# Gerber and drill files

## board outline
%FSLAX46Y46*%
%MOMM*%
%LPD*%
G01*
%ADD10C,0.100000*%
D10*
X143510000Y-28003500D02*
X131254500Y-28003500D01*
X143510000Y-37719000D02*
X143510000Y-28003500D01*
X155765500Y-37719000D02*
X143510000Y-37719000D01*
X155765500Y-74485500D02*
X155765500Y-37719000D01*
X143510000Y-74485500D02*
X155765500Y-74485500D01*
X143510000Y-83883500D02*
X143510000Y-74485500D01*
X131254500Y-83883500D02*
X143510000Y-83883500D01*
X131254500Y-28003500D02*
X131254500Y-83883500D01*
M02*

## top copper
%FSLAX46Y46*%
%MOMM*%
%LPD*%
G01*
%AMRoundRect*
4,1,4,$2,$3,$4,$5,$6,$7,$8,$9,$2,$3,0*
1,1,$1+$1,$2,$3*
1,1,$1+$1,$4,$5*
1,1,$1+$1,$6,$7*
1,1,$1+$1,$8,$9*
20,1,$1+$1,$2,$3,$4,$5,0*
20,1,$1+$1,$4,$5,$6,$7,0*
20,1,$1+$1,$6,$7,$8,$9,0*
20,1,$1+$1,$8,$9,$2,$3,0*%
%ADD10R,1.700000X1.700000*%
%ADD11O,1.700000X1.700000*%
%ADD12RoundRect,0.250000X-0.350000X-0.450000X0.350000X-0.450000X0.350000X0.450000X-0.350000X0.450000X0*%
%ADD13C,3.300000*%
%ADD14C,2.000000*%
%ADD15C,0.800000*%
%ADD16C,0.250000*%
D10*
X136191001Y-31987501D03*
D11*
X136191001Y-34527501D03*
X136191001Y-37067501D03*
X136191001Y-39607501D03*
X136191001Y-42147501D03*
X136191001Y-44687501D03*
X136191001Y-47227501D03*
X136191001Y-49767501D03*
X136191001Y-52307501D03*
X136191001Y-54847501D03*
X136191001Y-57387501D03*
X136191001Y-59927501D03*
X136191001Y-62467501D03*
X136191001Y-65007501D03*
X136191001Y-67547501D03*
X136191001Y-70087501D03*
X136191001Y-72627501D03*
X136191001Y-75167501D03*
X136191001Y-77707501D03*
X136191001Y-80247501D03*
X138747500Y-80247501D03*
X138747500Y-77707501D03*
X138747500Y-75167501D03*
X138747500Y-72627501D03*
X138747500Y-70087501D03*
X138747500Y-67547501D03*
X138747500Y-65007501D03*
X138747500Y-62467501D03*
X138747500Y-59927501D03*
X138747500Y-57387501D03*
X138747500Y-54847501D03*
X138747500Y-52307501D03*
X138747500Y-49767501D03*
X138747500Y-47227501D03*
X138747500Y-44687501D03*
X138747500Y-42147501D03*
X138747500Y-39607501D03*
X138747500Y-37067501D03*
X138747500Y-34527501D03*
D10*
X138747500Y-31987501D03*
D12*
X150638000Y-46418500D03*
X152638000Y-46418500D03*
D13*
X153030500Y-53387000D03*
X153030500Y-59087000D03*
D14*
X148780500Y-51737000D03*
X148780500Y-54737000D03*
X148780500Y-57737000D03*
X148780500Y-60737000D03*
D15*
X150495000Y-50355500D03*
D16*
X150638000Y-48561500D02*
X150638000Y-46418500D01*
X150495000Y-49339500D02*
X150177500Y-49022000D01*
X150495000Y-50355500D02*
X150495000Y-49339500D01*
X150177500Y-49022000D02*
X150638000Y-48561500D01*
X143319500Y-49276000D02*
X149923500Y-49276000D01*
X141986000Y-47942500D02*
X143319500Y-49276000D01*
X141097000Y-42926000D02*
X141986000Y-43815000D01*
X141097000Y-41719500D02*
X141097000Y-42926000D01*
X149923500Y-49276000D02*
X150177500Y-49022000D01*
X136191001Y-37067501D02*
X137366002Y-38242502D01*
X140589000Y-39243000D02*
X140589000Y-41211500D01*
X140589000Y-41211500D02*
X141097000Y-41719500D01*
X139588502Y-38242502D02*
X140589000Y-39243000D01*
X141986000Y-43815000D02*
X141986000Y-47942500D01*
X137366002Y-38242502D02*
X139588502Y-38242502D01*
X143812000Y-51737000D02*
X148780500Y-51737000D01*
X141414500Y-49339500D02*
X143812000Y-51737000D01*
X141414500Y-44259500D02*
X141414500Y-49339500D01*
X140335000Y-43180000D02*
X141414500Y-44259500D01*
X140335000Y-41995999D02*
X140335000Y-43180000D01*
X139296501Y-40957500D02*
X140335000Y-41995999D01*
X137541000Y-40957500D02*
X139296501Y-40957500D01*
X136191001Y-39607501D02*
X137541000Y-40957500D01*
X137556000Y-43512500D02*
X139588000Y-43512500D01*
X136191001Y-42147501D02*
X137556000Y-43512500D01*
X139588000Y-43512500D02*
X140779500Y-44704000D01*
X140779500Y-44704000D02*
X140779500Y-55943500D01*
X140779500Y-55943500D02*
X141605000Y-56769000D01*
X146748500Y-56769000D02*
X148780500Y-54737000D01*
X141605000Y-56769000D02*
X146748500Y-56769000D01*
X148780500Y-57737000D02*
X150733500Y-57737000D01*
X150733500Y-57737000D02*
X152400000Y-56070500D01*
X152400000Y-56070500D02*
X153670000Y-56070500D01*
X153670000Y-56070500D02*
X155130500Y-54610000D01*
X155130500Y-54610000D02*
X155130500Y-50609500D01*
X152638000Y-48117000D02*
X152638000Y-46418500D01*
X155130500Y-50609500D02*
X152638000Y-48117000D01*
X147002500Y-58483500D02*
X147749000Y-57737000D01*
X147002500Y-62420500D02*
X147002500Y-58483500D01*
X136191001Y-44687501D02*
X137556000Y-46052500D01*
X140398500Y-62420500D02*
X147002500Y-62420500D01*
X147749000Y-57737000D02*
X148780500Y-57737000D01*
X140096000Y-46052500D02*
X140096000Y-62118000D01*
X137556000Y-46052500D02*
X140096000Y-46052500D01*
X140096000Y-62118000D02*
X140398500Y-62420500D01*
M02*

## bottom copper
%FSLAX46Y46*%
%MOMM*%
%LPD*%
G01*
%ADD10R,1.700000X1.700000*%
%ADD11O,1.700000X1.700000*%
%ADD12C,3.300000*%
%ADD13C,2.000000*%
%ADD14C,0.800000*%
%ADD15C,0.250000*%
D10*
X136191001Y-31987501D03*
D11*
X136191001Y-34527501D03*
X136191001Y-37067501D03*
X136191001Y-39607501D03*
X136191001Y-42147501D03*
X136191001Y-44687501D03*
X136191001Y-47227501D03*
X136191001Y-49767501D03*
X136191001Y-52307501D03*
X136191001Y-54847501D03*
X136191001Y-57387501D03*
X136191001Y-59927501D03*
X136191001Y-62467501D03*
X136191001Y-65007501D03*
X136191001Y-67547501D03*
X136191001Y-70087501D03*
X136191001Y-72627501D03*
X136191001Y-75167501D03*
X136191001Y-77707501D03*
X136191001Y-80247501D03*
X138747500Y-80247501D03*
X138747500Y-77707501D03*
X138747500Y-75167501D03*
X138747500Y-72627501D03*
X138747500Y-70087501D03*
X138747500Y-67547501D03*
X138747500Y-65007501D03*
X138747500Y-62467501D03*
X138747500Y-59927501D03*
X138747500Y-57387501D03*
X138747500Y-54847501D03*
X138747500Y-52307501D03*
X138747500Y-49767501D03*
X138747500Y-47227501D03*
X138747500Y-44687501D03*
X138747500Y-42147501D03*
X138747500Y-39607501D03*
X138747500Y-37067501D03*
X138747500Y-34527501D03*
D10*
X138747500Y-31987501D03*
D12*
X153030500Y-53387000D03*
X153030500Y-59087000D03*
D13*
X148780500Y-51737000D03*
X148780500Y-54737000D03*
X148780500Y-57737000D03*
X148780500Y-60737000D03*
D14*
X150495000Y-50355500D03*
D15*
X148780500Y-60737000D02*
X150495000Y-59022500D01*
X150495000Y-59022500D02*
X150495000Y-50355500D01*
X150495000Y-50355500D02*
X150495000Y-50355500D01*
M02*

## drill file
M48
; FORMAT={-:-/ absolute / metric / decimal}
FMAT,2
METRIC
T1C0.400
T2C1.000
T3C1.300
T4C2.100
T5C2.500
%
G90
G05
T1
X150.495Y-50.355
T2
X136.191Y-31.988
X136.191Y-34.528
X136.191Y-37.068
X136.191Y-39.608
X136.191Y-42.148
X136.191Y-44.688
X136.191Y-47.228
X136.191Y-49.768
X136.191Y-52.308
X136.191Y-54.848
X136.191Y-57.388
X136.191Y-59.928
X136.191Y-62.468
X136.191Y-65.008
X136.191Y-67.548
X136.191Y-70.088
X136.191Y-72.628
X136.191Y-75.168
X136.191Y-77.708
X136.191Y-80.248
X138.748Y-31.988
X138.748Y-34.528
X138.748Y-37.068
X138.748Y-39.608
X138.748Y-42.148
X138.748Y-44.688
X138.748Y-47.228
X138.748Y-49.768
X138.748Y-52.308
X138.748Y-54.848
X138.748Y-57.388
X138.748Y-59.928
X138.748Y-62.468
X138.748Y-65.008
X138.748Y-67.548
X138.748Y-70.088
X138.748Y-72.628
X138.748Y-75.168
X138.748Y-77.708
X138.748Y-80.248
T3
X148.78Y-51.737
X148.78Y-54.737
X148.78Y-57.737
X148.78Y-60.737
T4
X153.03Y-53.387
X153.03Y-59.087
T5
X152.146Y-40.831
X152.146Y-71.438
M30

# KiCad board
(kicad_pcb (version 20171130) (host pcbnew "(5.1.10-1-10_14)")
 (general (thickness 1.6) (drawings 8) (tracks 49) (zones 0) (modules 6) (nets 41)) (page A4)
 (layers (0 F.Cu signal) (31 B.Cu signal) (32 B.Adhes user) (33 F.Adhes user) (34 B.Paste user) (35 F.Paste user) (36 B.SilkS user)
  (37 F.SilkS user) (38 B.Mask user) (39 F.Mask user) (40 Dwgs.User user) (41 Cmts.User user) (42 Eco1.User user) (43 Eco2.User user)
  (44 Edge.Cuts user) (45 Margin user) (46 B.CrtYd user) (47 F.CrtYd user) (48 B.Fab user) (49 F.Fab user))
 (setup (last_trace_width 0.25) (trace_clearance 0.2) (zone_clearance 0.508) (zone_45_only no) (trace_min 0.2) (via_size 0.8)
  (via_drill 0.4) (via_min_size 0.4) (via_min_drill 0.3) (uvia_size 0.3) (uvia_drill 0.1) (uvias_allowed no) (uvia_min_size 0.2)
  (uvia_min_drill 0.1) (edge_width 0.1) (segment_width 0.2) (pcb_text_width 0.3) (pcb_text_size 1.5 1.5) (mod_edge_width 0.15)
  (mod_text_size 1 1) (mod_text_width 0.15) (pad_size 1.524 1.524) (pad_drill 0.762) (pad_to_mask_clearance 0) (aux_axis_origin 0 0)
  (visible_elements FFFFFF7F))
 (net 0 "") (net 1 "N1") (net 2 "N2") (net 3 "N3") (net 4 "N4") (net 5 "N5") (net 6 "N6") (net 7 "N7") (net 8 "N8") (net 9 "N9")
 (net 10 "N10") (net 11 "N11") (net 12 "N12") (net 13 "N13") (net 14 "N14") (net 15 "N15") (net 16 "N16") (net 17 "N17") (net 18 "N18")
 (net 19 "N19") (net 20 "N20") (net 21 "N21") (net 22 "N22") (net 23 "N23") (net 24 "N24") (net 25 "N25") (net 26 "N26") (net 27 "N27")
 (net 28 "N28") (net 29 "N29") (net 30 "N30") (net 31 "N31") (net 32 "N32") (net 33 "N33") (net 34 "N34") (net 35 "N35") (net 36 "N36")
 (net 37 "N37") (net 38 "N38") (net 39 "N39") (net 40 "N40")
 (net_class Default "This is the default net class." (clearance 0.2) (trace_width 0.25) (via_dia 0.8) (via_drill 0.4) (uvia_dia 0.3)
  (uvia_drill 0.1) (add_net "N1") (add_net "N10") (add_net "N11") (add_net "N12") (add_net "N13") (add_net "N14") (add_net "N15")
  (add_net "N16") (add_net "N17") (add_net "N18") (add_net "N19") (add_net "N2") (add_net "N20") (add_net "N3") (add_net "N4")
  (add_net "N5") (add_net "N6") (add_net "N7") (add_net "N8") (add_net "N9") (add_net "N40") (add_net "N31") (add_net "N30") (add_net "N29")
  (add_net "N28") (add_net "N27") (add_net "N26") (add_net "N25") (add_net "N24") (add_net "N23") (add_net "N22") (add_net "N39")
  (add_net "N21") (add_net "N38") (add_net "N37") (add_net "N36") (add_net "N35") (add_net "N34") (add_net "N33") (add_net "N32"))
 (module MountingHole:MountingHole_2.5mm (layer F.Cu) (at 152.146 71.4375)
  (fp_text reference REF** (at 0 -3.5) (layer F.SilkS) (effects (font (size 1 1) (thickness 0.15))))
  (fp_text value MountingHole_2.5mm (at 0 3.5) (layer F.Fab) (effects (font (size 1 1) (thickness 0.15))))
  (pad 1 np_thru_hole circle (at 0 0) (size 2.5 2.5) (drill 2.5) (layers *.Cu *.Mask)))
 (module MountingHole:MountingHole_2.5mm (layer F.Cu) (at 152.146 40.8305)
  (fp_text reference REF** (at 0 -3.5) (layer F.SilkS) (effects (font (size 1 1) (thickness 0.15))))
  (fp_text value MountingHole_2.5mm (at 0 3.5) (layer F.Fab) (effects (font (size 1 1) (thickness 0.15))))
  (pad 1 np_thru_hole circle (at 0 0) (size 2.5 2.5) (drill 2.5) (layers *.Cu *.Mask)))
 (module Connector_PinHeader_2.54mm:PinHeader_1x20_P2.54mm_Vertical (layer F.Cu) (at 136.191001 31.987501)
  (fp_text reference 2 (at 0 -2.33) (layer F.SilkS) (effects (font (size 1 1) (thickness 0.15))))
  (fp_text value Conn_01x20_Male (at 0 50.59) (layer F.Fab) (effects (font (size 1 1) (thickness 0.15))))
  (pad 1 thru_hole rect (at 0 0) (size 1.7 1.7) (drill 1) (layers *.Cu *.Mask) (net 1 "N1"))
  (pad 2 thru_hole oval (at 0 2.54) (size 1.7 1.7) (drill 1) (layers *.Cu *.Mask) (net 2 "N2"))
  (pad 3 thru_hole oval (at 0 5.08) (size 1.7 1.7) (drill 1) (layers *.Cu *.Mask) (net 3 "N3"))
  (pad 4 thru_hole oval (at 0 7.62) (size 1.7 1.7) (drill 1) (layers *.Cu *.Mask) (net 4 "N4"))
  (pad 5 thru_hole oval (at 0 10.16) (size 1.7 1.7) (drill 1) (layers *.Cu *.Mask) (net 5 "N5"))
  (pad 6 thru_hole oval (at 0 12.7) (size 1.7 1.7) (drill 1) (layers *.Cu *.Mask) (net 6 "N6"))
  (pad 7 thru_hole oval (at 0 15.24) (size 1.7 1.7) (drill 1) (layers *.Cu *.Mask) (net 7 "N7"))
  (pad 8 thru_hole oval (at 0 17.78) (size 1.7 1.7) (drill 1) (layers *.Cu *.Mask) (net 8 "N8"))
  (pad 9 thru_hole oval (at 0 20.32) (size 1.7 1.7) (drill 1) (layers *.Cu *.Mask) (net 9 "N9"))
  (pad 10 thru_hole oval (at 0 22.86) (size 1.7 1.7) (drill 1) (layers *.Cu *.Mask) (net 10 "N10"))
  (pad 11 thru_hole oval (at 0 25.4) (size 1.7 1.7) (drill 1) (layers *.Cu *.Mask) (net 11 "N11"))
  (pad 12 thru_hole oval (at 0 27.94) (size 1.7 1.7) (drill 1) (layers *.Cu *.Mask) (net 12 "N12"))
  (pad 13 thru_hole oval (at 0 30.48) (size 1.7 1.7) (drill 1) (layers *.Cu *.Mask) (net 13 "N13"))
  (pad 14 thru_hole oval (at 0 33.02) (size 1.7 1.7) (drill 1) (layers *.Cu *.Mask) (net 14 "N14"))
  (pad 15 thru_hole oval (at 0 35.56) (size 1.7 1.7) (drill 1) (layers *.Cu *.Mask) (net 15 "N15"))
  (pad 16 thru_hole oval (at 0 38.1) (size 1.7 1.7) (drill 1) (layers *.Cu *.Mask) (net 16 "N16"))
  (pad 17 thru_hole oval (at 0 40.64) (size 1.7 1.7) (drill 1) (layers *.Cu *.Mask) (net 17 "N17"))
  (pad 18 thru_hole oval (at 0 43.18) (size 1.7 1.7) (drill 1) (layers *.Cu *.Mask) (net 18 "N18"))
  (pad 19 thru_hole oval (at 0 45.72) (size 1.7 1.7) (drill 1) (layers *.Cu *.Mask) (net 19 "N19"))
  (pad 20 thru_hole oval (at 0 48.26) (size 1.7 1.7) (drill 1) (layers *.Cu *.Mask) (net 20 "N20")))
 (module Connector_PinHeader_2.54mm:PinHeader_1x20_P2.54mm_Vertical (layer F.Cu) (at 138.7475 31.987501)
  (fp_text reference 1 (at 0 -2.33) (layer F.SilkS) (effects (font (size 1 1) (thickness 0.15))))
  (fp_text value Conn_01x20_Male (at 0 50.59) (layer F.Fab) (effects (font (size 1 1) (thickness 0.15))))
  (pad 20 thru_hole oval (at 0 48.26) (size 1.7 1.7) (drill 1) (layers *.Cu *.Mask) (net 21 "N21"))
  (pad 19 thru_hole oval (at 0 45.72) (size 1.7 1.7) (drill 1) (layers *.Cu *.Mask) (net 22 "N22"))
  (pad 18 thru_hole oval (at 0 43.18) (size 1.7 1.7) (drill 1) (layers *.Cu *.Mask) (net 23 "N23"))
  (pad 17 thru_hole oval (at 0 40.64) (size 1.7 1.7) (drill 1) (layers *.Cu *.Mask) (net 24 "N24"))
  (pad 16 thru_hole oval (at 0 38.1) (size 1.7 1.7) (drill 1) (layers *.Cu *.Mask) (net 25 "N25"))
  (pad 15 thru_hole oval (at 0 35.56) (size 1.7 1.7) (drill 1) (layers *.Cu *.Mask) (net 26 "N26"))
  (pad 14 thru_hole oval (at 0 33.02) (size 1.7 1.7) (drill 1) (layers *.Cu *.Mask) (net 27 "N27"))
  (pad 13 thru_hole oval (at 0 30.48) (size 1.7 1.7) (drill 1) (layers *.Cu *.Mask) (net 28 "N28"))
  (pad 12 thru_hole oval (at 0 27.94) (size 1.7 1.7) (drill 1) (layers *.Cu *.Mask) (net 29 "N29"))
  (pad 11 thru_hole oval (at 0 25.4) (size 1.7 1.7) (drill 1) (layers *.Cu *.Mask) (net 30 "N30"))
  (pad 10 thru_hole oval (at 0 22.86) (size 1.7 1.7) (drill 1) (layers *.Cu *.Mask) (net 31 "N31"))
  (pad 9 thru_hole oval (at 0 20.32) (size 1.7 1.7) (drill 1) (layers *.Cu *.Mask) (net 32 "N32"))
  (pad 8 thru_hole oval (at 0 17.78) (size 1.7 1.7) (drill 1) (layers *.Cu *.Mask) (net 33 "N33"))
  (pad 7 thru_hole oval (at 0 15.24) (size 1.7 1.7) (drill 1) (layers *.Cu *.Mask) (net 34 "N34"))
  (pad 6 thru_hole oval (at 0 12.7) (size 1.7 1.7) (drill 1) (layers *.Cu *.Mask) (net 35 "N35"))
  (pad 5 thru_hole oval (at 0 10.16) (size 1.7 1.7) (drill 1) (layers *.Cu *.Mask) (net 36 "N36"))
  (pad 4 thru_hole oval (at 0 7.62) (size 1.7 1.7) (drill 1) (layers *.Cu *.Mask) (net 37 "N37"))
  (pad 3 thru_hole oval (at 0 5.08) (size 1.7 1.7) (drill 1) (layers *.Cu *.Mask) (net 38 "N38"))
  (pad 2 thru_hole oval (at 0 2.54) (size 1.7 1.7) (drill 1) (layers *.Cu *.Mask) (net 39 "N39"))
  (pad 1 thru_hole rect (at 0 0) (size 1.7 1.7) (drill 1) (layers *.Cu *.Mask) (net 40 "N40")))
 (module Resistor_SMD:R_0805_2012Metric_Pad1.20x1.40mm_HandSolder (layer F.Cu) (at 151.638 46.4185)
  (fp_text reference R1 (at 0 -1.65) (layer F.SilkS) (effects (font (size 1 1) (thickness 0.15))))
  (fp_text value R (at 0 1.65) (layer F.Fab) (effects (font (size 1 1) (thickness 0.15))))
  (pad 1 smd roundrect (at -1 0) (size 1.2 1.4) (layers F.Cu F.Paste F.Mask) (roundrect_rratio 0.208333) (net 3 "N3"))
  (pad 2 smd roundrect (at 1 0) (size 1.2 1.4) (layers F.Cu F.Paste F.Mask) (roundrect_rratio 0.208333) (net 6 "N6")))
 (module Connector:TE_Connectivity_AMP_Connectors (layer B.Cu) (at 153.0305 53.887 270)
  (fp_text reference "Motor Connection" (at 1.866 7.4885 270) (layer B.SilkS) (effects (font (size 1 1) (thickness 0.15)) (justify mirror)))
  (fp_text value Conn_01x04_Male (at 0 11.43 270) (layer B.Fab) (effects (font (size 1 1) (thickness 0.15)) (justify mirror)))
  (pad 5 thru_hole circle (at -0.5 0 270) (size 3.3 3.3) (drill 2.1) (layers *.Cu *.Mask))
  (pad 6 thru_hole circle (at 5.2 0 270) (size 3.3 3.3) (drill 2.1) (layers *.Cu *.Mask))
  (pad 1 thru_hole circle (at -2.15 4.25 270) (size 2 2) (drill 1.3) (layers *.Cu *.Mask) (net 4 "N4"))
  (pad 2 thru_hole circle (at 0.85 4.25 270) (size 2 2) (drill 1.3) (layers *.Cu *.Mask) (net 5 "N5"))
  (pad 3 thru_hole circle (at 3.85 4.25 270) (size 2 2) (drill 1.3) (layers *.Cu *.Mask) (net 6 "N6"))
  (pad 4 thru_hole circle (at 6.85 4.25 270) (size 2 2) (drill 1.3) (layers *.Cu *.Mask) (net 3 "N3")))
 (gr_line (start 143.51 28.0035) (end 131.2545 28.0035) (layer Edge.Cuts) (width 0.1))
 (gr_line (start 143.51 37.719) (end 143.51 28.0035) (layer Edge.Cuts) (width 0.1))
 (gr_line (start 155.7655 37.719) (end 143.51 37.719) (layer Edge.Cuts) (width 0.1))
 (gr_line (start 155.7655 74.4855) (end 155.7655 37.719) (layer Edge.Cuts) (width 0.1))
 (gr_line (start 143.51 74.4855) (end 155.7655 74.4855) (layer Edge.Cuts) (width 0.1))
 (gr_line (start 143.51 83.8835) (end 143.51 74.4855) (layer Edge.Cuts) (width 0.1))
 (gr_line (start 131.2545 83.8835) (end 143.51 83.8835) (layer Edge.Cuts) (width 0.1))
 (gr_line (start 131.2545 28.0035) (end 131.2545 83.8835) (layer Edge.Cuts) (width 0.1))
 (segment (start 150.638 48.5615) (end 150.638 46.4185) (width 0.25) (layer F.Cu) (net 3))
 (segment (start 148.7805 60.737) (end 150.495 59.0225) (width 0.25) (layer B.Cu) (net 3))
 (segment (start 150.495 59.0225) (end 150.495 50.3555) (width 0.25) (layer B.Cu) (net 3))
 (segment (start 150.495 50.3555) (end 150.495 50.3555) (width 0.25) (layer B.Cu) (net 3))
 (via (at 150.495 50.3555) (size 0.8) (drill 0.4) (layers F.Cu B.Cu) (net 3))
 (segment (start 150.495 49.3395) (end 150.1775 49.022) (width 0.25) (layer F.Cu) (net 3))
 (segment (start 150.495 50.3555) (end 150.495 49.3395) (width 0.25) (layer F.Cu) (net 3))
 (segment (start 150.1775 49.022) (end 150.638 48.5615) (width 0.25) (layer F.Cu) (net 3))
 (segment (start 143.3195 49.276) (end 149.9235 49.276) (width 0.25) (layer F.Cu) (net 3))
 (segment (start 141.986 47.9425) (end 143.3195 49.276) (width 0.25) (layer F.Cu) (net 3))
 (segment (start 141.097 42.926) (end 141.986 43.815) (width 0.25) (layer F.Cu) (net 3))
 (segment (start 141.097 41.7195) (end 141.097 42.926) (width 0.25) (layer F.Cu) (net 3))
 (segment (start 149.9235 49.276) (end 150.1775 49.022) (width 0.25) (layer F.Cu) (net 3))
 (segment (start 136.191001 37.067501) (end 137.366002 38.242502) (width 0.25) (layer F.Cu) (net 3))
 (segment (start 140.589 39.243) (end 140.589 41.2115) (width 0.25) (layer F.Cu) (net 3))
 (segment (start 140.589 41.2115) (end 141.097 41.7195) (width 0.25) (layer F.Cu) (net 3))
 (segment (start 139.588502 38.242502) (end 140.589 39.243) (width 0.25) (layer F.Cu) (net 3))
 (segment (start 141.986 43.815) (end 141.986 47.9425) (width 0.25) (layer F.Cu) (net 3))
 (segment (start 137.366002 38.242502) (end 139.588502 38.242502) (width 0.25) (layer F.Cu) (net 3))
 (segment (start 143.812 51.737) (end 148.7805 51.737) (width 0.25) (layer F.Cu) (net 4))
 (segment (start 141.4145 49.3395) (end 143.812 51.737) (width 0.25) (layer F.Cu) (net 4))
 (segment (start 141.4145 44.2595) (end 141.4145 49.3395) (width 0.25) (layer F.Cu) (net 4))
 (segment (start 140.335 43.18) (end 141.4145 44.2595) (width 0.25) (layer F.Cu) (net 4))
 (segment (start 140.335 41.995999) (end 140.335 43.18) (width 0.25) (layer F.Cu) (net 4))
 (segment (start 139.296501 40.9575) (end 140.335 41.995999) (width 0.25) (layer F.Cu) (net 4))
 (segment (start 137.541 40.9575) (end 139.296501 40.9575) (width 0.25) (layer F.Cu) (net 4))
 (segment (start 136.191001 39.607501) (end 137.541 40.9575) (width 0.25) (layer F.Cu) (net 4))
 (segment (start 137.556 43.5125) (end 139.588 43.5125) (width 0.25) (layer F.Cu) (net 5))
 (segment (start 136.191001 42.147501) (end 137.556 43.5125) (width 0.25) (layer F.Cu) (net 5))
 (segment (start 139.588 43.5125) (end 140.7795 44.704) (width 0.25) (layer F.Cu) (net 5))
 (segment (start 140.7795 44.704) (end 140.7795 55.9435) (width 0.25) (layer F.Cu) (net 5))
 (segment (start 140.7795 55.9435) (end 141.605 56.769) (width 0.25) (layer F.Cu) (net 5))
 (segment (start 146.7485 56.769) (end 148.7805 54.737) (width 0.25) (layer F.Cu) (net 5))
 (segment (start 141.605 56.769) (end 146.7485 56.769) (width 0.25) (layer F.Cu) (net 5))
 (segment (start 148.7805 57.737) (end 150.7335 57.737) (width 0.25) (layer F.Cu) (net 6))
 (segment (start 150.7335 57.737) (end 152.4 56.0705) (width 0.25) (layer F.Cu) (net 6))
 (segment (start 152.4 56.0705) (end 153.67 56.0705) (width 0.25) (layer F.Cu) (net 6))
 (segment (start 153.67 56.0705) (end 155.1305 54.61) (width 0.25) (layer F.Cu) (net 6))
 (segment (start 155.1305 54.61) (end 155.1305 50.6095) (width 0.25) (layer F.Cu) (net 6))
 (segment (start 152.638 48.117) (end 152.638 46.4185) (width 0.25) (layer F.Cu) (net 6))
 (segment (start 155.1305 50.6095) (end 152.638 48.117) (width 0.25) (layer F.Cu) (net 6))
 (segment (start 147.0025 58.4835) (end 147.749 57.737) (width 0.25) (layer F.Cu) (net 6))
 (segment (start 147.0025 62.4205) (end 147.0025 58.4835) (width 0.25) (layer F.Cu) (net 6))
 (segment (start 136.191001 44.687501) (end 137.556 46.0525) (width 0.25) (layer F.Cu) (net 6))
 (segment (start 140.3985 62.4205) (end 147.0025 62.4205) (width 0.25) (layer F.Cu) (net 6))
 (segment (start 147.749 57.737) (end 148.7805 57.737) (width 0.25) (layer F.Cu) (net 6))
 (segment (start 140.096 46.0525) (end 140.096 62.118) (width 0.25) (layer F.Cu) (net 6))
 (segment (start 137.556 46.0525) (end 140.096 46.0525) (width 0.25) (layer F.Cu) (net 6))
 (segment (start 140.096 62.118) (end 140.3985 62.4205) (width 0.25) (layer F.Cu) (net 6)))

